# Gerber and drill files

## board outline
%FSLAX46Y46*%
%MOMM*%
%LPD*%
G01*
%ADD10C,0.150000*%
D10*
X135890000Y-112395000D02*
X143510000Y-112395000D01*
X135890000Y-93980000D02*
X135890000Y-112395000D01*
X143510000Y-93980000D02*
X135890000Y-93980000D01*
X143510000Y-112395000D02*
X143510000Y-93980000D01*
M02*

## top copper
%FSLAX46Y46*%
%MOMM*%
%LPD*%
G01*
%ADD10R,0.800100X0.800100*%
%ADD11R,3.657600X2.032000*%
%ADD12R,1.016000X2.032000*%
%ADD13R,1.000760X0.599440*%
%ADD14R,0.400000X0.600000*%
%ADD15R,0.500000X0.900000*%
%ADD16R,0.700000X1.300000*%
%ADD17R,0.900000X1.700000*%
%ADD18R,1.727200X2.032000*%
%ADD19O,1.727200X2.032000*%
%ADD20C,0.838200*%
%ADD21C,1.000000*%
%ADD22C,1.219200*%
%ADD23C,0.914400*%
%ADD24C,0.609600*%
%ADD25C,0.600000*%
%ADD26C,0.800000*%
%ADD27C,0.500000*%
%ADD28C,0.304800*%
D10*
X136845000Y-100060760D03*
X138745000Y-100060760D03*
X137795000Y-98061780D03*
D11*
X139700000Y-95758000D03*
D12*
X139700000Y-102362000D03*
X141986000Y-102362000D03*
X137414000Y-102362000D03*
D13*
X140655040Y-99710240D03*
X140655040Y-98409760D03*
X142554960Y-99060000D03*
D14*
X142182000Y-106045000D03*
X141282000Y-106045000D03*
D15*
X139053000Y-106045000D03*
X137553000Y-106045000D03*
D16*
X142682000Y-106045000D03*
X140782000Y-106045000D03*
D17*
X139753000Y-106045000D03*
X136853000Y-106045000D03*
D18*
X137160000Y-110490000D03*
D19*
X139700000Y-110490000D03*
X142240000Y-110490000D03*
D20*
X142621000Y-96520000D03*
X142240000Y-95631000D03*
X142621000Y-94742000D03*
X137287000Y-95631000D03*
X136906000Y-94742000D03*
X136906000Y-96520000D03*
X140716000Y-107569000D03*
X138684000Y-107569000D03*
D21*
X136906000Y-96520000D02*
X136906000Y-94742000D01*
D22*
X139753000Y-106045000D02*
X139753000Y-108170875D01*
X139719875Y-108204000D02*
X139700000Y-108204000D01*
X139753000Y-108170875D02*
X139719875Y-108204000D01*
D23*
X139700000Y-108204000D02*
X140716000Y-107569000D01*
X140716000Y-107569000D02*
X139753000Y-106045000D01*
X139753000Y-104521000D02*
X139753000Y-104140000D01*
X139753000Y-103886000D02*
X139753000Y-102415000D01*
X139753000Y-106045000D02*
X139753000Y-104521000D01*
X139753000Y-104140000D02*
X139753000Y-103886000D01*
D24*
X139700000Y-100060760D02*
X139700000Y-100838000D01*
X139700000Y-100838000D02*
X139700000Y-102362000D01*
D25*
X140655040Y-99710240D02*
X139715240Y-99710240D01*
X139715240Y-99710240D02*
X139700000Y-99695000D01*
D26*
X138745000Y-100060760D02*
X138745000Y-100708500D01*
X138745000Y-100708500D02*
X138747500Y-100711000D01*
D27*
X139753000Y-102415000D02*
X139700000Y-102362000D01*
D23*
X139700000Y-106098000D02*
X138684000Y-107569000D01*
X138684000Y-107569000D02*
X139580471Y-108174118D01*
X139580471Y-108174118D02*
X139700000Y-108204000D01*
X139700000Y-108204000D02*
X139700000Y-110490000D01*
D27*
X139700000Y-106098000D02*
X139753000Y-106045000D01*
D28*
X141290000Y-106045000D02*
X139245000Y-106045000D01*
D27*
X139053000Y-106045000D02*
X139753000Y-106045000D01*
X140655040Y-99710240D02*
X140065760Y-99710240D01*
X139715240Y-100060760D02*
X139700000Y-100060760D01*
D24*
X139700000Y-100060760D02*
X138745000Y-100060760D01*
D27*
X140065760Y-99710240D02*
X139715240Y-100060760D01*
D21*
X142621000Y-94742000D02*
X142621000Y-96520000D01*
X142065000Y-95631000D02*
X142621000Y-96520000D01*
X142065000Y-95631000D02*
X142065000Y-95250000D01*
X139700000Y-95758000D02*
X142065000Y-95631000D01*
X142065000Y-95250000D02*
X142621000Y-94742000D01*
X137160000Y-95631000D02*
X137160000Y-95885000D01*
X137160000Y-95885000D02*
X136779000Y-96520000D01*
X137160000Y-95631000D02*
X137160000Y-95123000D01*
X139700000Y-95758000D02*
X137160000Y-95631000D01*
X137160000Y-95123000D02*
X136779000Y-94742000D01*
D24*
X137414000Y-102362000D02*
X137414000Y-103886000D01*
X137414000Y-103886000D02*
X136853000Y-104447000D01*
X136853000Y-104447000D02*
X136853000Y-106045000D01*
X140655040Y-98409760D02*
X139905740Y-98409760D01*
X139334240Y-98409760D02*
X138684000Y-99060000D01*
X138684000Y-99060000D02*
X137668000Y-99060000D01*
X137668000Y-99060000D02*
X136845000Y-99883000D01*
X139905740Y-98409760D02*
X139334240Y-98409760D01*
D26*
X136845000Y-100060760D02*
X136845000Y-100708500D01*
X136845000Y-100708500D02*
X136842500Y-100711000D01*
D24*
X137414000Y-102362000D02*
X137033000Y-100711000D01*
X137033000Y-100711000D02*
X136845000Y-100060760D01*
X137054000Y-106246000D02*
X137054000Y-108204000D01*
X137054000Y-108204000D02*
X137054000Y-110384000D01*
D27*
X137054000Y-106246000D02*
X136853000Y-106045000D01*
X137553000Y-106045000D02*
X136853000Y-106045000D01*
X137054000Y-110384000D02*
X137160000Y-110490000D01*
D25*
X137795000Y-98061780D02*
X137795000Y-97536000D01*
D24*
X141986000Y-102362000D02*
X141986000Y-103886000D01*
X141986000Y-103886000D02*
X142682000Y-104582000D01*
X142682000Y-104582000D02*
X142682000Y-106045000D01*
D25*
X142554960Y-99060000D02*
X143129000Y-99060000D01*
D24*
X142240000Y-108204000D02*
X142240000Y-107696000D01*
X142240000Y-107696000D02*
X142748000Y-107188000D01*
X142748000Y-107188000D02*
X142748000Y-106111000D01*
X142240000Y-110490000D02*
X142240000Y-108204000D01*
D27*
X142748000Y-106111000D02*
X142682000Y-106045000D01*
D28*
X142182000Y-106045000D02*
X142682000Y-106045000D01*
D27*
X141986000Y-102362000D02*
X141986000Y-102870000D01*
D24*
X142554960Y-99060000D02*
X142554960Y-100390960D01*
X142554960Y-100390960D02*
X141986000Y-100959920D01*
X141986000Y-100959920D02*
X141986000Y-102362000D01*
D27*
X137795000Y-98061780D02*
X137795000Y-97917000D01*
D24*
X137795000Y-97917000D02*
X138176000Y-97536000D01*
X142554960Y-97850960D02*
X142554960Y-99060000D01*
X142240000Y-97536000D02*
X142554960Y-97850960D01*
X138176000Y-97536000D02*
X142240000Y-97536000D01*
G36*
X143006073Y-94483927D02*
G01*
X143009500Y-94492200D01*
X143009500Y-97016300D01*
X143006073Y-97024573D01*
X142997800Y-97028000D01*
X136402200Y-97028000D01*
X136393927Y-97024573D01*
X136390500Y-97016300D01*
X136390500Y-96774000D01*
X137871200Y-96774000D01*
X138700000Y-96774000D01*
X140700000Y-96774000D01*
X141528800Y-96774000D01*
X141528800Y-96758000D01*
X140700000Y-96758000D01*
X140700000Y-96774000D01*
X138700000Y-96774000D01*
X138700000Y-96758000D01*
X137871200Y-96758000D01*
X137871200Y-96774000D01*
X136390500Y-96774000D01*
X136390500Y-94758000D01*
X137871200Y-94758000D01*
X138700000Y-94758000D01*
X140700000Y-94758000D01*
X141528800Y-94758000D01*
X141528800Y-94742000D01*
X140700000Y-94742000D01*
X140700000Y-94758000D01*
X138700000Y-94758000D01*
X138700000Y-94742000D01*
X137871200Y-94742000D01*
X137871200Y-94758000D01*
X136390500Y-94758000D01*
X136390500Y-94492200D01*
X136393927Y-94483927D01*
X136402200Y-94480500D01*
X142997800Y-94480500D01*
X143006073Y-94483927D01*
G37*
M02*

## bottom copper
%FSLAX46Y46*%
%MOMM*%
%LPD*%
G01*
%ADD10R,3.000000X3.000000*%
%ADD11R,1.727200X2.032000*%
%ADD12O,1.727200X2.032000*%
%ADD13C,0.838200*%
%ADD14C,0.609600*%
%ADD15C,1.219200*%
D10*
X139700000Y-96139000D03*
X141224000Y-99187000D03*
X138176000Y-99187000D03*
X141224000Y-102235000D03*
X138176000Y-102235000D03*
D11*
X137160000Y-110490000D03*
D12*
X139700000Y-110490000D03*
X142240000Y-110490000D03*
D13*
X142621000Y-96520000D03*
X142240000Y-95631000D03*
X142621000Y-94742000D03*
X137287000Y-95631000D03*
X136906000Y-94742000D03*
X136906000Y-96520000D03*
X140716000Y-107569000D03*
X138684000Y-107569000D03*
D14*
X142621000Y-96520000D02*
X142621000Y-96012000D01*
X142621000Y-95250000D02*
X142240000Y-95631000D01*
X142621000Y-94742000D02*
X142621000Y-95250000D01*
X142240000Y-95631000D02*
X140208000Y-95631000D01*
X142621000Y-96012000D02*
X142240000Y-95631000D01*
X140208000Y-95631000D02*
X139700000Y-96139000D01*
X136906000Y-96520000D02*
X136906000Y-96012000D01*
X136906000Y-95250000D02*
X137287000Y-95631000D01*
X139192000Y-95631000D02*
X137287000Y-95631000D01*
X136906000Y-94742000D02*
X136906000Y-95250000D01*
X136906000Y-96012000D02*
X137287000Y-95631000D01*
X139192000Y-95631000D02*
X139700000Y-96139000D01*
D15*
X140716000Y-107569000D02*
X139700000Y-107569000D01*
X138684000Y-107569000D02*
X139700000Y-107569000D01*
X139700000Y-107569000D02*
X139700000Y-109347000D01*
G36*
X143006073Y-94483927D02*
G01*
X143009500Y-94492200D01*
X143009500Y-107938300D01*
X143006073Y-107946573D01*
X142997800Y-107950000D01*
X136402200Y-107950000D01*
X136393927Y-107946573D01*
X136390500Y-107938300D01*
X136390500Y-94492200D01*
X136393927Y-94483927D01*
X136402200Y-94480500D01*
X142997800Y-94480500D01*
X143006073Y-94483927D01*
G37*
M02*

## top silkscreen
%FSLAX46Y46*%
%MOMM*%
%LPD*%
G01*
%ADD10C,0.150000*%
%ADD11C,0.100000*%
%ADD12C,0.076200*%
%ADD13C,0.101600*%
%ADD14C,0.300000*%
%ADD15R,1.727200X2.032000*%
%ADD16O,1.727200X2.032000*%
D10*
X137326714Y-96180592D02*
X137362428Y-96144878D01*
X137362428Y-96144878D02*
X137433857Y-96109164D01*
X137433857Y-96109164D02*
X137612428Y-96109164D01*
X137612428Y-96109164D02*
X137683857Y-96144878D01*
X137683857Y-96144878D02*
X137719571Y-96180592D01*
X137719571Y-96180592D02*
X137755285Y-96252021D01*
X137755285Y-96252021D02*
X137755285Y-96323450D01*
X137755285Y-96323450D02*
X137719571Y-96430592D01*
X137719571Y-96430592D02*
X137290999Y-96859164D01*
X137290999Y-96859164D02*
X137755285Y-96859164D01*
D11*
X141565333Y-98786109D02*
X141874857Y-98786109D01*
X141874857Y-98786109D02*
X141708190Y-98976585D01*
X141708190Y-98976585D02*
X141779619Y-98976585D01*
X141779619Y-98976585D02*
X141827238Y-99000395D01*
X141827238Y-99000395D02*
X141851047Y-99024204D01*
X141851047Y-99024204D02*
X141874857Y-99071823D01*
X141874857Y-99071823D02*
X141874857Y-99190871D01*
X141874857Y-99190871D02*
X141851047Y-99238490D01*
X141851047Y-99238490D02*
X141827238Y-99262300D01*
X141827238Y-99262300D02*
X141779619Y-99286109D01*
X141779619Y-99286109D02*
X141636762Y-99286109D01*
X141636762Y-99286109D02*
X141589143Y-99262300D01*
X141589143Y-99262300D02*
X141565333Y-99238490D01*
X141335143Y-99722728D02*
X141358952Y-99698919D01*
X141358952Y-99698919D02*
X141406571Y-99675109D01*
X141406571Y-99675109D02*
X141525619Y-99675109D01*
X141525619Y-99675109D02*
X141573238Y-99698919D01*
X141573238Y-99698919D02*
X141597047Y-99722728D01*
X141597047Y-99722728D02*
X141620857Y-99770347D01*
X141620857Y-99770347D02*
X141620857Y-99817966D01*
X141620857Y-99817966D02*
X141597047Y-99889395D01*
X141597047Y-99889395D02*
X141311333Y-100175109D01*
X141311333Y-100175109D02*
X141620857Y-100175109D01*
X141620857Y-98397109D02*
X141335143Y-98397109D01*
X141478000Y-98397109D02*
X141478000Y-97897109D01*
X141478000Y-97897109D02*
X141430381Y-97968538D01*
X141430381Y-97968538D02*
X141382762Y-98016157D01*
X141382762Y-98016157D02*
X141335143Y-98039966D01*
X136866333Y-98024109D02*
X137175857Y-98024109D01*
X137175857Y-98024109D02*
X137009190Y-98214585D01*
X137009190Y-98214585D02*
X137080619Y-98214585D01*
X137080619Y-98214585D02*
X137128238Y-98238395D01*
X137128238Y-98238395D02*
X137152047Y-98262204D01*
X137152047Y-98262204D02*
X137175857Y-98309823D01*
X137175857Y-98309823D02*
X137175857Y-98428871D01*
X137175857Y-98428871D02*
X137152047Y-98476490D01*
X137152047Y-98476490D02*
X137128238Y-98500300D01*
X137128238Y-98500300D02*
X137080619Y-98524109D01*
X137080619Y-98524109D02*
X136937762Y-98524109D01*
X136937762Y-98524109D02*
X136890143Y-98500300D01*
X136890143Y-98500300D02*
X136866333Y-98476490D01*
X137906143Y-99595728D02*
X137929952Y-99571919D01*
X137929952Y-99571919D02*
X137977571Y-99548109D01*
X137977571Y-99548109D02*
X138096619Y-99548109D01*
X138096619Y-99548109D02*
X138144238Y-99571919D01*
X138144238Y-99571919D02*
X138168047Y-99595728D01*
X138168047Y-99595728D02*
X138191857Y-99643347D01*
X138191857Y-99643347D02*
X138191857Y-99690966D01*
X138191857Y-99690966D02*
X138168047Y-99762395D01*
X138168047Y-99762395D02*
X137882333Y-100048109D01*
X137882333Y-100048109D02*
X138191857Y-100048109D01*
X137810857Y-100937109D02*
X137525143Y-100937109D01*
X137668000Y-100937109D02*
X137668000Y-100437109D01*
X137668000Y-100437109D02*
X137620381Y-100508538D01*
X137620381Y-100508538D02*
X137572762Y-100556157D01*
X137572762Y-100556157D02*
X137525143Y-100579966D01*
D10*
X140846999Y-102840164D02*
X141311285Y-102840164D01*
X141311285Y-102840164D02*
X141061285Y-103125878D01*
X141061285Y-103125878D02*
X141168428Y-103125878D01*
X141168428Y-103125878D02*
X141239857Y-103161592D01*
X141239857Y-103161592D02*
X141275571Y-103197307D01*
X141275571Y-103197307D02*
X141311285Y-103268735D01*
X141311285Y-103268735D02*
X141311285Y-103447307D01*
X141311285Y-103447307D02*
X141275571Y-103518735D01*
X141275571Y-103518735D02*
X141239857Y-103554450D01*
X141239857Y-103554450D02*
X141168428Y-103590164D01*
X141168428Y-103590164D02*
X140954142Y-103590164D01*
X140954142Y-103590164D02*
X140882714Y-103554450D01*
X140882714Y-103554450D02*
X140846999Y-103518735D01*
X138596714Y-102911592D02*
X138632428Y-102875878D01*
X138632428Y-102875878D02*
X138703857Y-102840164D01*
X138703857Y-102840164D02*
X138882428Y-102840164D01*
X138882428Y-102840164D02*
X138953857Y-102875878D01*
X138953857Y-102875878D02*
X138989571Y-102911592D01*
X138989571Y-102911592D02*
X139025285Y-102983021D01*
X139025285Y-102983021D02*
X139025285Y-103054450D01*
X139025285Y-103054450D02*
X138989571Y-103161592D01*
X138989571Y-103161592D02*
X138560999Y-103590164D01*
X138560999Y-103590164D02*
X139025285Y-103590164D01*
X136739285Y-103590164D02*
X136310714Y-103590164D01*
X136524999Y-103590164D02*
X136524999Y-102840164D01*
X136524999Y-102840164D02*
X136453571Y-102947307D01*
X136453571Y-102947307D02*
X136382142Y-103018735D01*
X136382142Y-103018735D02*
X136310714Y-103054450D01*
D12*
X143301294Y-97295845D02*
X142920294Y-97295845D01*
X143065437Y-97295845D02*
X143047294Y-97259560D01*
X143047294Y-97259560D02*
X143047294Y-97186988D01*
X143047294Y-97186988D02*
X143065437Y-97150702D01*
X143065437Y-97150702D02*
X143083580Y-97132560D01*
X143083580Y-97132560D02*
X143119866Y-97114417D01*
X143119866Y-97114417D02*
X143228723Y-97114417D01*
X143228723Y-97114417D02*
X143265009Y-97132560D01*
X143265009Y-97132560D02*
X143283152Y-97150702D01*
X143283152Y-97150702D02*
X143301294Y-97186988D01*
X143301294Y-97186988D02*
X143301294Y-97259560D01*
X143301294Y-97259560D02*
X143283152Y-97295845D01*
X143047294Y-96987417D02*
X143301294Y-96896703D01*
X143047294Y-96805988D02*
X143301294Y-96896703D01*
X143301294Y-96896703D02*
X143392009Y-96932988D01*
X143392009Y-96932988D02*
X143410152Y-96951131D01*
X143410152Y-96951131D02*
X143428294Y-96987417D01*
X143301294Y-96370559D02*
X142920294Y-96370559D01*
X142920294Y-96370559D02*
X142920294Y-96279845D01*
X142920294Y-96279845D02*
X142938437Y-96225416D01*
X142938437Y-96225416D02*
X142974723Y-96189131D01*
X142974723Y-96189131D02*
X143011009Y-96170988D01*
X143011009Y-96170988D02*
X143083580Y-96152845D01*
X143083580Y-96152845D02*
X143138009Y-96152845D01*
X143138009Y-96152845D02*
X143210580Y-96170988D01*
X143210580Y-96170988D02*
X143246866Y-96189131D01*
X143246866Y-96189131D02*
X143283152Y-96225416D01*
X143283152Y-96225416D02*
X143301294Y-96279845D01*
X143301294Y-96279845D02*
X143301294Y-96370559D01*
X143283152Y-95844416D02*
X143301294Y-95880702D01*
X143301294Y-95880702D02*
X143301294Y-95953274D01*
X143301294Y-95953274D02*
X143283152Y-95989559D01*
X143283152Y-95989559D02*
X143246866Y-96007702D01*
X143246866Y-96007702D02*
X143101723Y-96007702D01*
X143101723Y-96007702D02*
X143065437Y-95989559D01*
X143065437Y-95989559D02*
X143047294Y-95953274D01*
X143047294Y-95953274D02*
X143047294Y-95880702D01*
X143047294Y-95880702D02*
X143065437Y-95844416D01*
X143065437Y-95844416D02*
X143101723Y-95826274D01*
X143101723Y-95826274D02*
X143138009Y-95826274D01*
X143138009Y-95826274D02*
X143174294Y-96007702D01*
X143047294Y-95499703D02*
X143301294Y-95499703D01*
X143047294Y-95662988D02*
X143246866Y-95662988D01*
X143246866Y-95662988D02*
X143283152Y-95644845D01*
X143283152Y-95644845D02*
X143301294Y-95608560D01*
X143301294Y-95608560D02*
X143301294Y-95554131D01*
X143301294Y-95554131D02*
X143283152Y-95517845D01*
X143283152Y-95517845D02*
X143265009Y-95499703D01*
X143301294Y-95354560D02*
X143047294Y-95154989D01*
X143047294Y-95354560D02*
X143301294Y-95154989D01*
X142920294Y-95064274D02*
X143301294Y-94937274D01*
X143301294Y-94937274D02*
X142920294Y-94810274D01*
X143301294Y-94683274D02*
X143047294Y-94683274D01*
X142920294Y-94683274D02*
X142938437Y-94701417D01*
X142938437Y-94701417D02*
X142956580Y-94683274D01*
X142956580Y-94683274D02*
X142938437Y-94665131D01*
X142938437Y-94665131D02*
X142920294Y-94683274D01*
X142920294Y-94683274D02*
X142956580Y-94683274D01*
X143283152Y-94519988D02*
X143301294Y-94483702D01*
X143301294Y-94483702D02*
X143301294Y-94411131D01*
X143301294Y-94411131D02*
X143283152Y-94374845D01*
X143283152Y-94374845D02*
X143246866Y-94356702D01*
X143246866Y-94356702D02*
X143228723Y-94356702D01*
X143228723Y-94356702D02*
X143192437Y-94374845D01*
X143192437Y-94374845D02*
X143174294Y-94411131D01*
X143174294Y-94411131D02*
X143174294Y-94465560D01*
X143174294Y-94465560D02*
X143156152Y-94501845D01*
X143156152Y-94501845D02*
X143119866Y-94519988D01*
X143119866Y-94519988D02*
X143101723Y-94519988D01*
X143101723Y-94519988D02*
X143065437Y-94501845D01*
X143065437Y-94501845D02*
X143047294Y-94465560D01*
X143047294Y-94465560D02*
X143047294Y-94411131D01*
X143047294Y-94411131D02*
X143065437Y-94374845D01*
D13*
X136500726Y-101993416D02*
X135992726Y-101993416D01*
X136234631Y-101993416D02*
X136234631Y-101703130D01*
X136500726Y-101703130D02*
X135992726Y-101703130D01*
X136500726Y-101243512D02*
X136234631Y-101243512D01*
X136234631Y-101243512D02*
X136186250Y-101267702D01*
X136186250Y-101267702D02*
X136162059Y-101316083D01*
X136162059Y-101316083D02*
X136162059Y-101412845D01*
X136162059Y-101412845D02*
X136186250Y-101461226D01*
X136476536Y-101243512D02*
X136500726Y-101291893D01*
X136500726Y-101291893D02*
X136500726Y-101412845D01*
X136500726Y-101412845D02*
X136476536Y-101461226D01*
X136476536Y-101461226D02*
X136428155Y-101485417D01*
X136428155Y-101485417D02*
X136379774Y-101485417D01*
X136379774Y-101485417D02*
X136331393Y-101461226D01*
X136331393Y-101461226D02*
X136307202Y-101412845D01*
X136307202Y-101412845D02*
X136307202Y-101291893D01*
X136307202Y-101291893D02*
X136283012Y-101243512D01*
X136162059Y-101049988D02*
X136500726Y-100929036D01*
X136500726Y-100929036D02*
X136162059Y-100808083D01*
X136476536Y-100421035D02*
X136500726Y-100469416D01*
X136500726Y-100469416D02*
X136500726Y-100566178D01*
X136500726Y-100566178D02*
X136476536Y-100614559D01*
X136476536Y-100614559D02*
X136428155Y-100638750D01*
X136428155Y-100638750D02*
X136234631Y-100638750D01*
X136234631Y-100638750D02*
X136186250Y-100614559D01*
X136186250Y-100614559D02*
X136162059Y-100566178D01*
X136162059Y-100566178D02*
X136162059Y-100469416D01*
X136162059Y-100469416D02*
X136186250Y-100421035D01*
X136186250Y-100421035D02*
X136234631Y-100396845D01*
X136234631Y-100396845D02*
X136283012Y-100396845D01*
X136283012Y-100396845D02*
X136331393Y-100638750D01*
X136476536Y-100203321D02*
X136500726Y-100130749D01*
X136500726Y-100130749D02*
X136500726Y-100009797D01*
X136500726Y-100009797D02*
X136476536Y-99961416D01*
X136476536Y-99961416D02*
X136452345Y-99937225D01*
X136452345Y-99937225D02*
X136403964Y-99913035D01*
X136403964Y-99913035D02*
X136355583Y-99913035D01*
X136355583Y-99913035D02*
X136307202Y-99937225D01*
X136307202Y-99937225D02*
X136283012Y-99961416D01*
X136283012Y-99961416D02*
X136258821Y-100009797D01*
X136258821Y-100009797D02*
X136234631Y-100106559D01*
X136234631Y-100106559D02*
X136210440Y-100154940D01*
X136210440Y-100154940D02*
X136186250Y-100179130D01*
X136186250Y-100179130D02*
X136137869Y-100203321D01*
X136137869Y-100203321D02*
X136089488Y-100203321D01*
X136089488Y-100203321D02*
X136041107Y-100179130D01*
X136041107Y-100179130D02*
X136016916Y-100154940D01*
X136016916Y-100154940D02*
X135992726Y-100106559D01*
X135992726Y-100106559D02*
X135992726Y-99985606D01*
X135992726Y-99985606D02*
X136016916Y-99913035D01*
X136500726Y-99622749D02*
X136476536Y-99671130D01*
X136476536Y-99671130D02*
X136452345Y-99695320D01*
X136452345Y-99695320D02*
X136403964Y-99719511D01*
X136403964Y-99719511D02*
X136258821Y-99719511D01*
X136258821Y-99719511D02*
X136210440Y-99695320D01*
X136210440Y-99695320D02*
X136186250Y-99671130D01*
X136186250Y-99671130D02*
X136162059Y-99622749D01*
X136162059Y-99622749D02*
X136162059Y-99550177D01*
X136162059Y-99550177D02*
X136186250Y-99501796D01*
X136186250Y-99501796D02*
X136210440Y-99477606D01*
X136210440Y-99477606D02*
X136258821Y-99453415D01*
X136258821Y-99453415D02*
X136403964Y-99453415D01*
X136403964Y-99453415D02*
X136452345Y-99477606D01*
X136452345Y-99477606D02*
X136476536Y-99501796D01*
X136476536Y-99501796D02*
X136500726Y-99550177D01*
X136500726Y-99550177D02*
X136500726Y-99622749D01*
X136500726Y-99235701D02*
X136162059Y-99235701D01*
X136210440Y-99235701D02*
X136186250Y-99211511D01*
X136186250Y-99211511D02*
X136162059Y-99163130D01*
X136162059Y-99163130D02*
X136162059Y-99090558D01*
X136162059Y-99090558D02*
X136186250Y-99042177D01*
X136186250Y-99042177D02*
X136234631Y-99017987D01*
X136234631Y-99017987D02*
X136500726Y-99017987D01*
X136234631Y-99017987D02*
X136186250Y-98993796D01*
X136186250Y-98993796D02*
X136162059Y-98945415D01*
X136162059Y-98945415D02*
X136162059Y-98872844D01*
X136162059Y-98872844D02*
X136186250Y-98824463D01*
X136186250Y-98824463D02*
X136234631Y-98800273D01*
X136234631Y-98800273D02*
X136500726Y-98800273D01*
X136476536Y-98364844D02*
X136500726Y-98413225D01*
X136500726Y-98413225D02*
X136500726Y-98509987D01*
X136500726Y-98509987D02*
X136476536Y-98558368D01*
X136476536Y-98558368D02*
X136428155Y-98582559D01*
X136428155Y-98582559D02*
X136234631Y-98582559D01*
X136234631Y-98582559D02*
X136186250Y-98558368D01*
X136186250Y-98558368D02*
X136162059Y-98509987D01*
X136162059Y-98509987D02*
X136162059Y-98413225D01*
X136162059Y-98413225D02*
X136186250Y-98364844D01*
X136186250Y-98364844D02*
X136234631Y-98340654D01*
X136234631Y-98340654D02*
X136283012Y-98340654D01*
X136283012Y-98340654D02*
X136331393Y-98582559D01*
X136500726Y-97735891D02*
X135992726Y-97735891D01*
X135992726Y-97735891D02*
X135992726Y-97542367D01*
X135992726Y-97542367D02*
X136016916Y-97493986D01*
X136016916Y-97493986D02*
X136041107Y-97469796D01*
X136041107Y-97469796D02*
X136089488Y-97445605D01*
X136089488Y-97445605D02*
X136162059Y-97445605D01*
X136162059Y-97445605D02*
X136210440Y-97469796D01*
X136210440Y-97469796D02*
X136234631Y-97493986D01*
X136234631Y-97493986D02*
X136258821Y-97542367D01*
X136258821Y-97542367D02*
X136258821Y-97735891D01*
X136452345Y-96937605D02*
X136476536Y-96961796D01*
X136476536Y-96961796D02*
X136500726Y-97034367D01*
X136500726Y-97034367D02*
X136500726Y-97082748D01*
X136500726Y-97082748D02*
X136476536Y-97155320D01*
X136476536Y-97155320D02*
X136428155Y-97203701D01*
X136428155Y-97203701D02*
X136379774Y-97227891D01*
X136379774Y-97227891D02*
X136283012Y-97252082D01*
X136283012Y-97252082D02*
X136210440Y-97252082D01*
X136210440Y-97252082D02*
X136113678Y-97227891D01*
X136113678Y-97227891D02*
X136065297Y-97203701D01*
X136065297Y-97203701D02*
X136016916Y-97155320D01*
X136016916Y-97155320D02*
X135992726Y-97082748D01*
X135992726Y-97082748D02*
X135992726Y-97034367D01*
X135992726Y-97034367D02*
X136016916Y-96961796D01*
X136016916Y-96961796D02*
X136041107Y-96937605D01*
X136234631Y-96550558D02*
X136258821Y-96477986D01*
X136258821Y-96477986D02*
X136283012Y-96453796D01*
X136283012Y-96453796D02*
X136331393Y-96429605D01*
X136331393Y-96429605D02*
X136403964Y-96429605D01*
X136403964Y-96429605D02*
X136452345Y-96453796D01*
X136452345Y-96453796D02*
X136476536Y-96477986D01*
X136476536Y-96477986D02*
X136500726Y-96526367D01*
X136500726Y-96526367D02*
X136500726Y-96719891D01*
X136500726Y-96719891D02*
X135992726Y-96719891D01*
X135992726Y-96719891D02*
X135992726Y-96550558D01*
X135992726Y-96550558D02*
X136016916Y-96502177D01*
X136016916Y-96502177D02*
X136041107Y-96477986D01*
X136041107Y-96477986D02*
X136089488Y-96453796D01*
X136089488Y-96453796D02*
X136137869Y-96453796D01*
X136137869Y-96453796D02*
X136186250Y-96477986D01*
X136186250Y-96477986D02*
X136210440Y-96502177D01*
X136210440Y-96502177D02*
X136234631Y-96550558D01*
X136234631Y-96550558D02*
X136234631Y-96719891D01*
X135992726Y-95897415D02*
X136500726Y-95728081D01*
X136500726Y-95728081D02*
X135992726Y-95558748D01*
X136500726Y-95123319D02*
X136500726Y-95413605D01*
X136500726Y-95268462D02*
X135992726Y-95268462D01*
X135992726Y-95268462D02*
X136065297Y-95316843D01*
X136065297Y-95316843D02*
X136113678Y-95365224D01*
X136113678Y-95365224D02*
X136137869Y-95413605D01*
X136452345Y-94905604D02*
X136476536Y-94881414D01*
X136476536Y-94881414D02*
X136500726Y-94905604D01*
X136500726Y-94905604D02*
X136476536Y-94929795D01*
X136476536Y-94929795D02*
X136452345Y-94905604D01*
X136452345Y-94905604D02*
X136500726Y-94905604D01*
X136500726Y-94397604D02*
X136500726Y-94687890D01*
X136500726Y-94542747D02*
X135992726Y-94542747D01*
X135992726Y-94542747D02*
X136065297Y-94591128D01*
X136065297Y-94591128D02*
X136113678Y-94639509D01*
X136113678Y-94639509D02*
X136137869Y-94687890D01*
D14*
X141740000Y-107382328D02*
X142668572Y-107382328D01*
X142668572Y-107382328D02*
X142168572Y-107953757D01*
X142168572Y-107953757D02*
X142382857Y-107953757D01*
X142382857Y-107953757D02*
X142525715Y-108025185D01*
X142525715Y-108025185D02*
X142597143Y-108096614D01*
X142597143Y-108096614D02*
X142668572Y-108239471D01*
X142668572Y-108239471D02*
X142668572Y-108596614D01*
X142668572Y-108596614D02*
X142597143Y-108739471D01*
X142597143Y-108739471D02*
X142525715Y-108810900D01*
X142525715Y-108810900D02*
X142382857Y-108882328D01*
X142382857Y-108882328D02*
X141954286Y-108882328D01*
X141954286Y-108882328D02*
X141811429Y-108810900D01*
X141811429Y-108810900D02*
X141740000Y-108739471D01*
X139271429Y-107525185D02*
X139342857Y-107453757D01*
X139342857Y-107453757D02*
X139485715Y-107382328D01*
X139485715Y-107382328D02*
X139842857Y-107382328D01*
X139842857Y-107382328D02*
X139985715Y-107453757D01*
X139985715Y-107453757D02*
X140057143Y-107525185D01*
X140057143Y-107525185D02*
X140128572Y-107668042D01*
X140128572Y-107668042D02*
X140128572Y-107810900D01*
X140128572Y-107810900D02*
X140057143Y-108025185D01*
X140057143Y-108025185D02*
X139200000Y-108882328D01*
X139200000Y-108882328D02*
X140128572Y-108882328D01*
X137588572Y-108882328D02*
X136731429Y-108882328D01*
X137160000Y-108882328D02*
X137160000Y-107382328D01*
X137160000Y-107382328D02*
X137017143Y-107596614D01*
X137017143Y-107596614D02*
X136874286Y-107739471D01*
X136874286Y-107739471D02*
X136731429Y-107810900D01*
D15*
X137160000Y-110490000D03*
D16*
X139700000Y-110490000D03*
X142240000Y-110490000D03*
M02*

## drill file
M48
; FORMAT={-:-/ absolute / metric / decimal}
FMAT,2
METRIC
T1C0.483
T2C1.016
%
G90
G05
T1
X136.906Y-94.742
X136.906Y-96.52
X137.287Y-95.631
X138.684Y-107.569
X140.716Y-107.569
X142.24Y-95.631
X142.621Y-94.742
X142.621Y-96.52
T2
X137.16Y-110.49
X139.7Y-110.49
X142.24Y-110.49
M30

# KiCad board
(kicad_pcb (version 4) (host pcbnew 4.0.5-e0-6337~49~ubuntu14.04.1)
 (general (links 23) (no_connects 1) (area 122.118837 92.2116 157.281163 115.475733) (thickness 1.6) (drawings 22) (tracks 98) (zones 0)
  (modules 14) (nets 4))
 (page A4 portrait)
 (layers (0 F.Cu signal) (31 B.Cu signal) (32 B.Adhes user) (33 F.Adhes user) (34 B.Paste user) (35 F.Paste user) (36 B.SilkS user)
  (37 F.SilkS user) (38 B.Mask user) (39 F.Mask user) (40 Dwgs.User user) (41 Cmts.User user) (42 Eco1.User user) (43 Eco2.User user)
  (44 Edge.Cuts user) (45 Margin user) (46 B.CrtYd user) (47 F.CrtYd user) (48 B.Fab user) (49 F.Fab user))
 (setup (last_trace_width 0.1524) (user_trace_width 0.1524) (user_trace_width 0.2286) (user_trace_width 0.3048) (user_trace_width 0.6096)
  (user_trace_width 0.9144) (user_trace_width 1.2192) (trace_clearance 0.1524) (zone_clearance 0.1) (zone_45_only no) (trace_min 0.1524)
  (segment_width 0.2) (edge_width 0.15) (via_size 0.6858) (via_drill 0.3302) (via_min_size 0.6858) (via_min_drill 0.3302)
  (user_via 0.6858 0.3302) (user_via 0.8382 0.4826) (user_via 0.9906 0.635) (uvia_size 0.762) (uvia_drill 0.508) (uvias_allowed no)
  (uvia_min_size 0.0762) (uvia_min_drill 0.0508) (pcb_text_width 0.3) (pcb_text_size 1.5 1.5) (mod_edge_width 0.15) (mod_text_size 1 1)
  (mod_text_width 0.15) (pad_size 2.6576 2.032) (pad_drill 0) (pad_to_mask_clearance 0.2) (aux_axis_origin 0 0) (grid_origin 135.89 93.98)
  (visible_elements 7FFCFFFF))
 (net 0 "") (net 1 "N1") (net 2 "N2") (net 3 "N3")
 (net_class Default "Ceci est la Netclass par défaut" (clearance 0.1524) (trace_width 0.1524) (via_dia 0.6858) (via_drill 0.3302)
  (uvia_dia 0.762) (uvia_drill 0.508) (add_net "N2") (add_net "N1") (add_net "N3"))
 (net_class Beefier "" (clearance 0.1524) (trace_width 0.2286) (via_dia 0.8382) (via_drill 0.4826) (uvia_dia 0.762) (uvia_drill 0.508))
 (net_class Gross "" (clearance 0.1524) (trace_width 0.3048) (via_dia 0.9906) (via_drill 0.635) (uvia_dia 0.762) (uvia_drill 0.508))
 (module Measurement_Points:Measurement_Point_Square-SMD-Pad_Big (layer B.Cu) (at 139.7 96.139)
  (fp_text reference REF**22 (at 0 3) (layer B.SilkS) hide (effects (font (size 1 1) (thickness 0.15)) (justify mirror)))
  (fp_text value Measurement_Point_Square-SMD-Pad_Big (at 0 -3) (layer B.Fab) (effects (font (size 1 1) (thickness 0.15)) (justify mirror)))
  (pad 1 smd rect (at 0 0) (size 3 3) (layers B.Cu B.Mask) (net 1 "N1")))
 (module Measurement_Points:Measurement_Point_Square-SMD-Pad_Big (layer B.Cu) (at 141.224 99.187)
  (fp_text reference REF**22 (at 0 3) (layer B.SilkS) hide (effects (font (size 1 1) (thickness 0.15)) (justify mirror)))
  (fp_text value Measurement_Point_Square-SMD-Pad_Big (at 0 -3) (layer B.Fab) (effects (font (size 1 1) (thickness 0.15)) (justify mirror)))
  (pad 1 smd rect (at 0 0) (size 3 3) (layers B.Cu B.Mask) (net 1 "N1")))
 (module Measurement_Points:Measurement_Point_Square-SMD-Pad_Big (layer B.Cu) (at 138.176 99.187) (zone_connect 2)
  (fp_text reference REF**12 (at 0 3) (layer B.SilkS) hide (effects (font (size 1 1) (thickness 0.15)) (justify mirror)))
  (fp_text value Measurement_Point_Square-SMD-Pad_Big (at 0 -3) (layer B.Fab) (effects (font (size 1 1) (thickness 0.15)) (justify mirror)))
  (pad 1 smd rect (at 0 0) (size 3 3) (layers B.Cu B.Mask) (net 1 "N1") (zone_connect 2)))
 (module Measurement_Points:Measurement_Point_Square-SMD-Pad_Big (layer B.Cu) (at 141.224 102.235)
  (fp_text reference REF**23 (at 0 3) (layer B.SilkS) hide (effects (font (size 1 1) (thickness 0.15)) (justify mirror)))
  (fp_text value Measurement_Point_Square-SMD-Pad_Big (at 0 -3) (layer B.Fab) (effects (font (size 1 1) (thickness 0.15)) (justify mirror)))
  (pad 1 smd rect (at 0 0) (size 3 3) (layers B.Cu B.Mask) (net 1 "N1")))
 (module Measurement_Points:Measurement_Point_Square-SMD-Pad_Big (layer B.Cu) (at 138.176 102.235) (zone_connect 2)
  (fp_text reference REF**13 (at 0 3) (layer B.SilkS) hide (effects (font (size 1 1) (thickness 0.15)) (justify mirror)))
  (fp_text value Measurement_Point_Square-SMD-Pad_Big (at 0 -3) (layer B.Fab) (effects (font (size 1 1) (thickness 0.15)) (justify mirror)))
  (pad 1 smd rect (at 0 0) (size 3 3) (layers B.Cu B.Mask) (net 1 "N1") (zone_connect 2)))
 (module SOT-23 (layer F.Cu) (at 137.795 99.06)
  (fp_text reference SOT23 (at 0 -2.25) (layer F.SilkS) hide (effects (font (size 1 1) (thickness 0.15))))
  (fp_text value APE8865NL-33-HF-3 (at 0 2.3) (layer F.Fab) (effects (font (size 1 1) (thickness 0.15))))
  (pad 1 smd rect (at -0.95 1.00076) (size 0.8001 0.8001) (layers F.Cu F.Paste F.Mask) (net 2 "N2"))
  (pad 2 smd rect (at 0.95 1.00076) (size 0.8001 0.8001) (layers F.Cu F.Paste F.Mask) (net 1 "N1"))
  (pad 3 smd rect (at 0 -0.99822) (size 0.8001 0.8001) (layers F.Cu F.Paste F.Mask) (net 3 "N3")))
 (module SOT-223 (layer F.Cu) (at 139.7 99.06)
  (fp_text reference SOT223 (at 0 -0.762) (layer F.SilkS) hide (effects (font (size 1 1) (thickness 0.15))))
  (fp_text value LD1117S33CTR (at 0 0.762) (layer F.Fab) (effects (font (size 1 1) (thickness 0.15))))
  (pad 4 smd rect (at 0 -3.302) (size 3.6576 2.032) (layers F.Cu F.Paste F.Mask) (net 1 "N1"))
  (pad 2 smd rect (at 0 3.302) (size 1.016 2.032) (layers F.Cu F.Paste F.Mask) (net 1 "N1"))
  (pad 3 smd rect (at 2.286 3.302) (size 1.016 2.032) (layers F.Cu F.Paste F.Mask) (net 3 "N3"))
  (pad 1 smd rect (at -2.286 3.302) (size 1.016 2.032) (layers F.Cu F.Paste F.Mask) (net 2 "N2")))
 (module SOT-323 (layer F.Cu) (at 141.605 99.06 90)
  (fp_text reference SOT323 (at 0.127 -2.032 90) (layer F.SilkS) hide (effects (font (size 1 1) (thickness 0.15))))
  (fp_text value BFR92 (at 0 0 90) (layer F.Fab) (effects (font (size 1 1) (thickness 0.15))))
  (pad 2 smd rect (at -0.65024 -0.94996 90) (size 0.59944 1.00076) (layers F.Cu F.Paste F.Mask) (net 1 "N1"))
  (pad 1 smd rect (at 0.65024 -0.94996 90) (size 0.59944 1.00076) (layers F.Cu F.Paste F.Mask) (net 2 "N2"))
  (pad 3 smd rect (at 0 0.94996 90) (size 0.59944 1.00076) (layers F.Cu F.Paste F.Mask) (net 3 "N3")))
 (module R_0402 (layer F.Cu) (at 141.732 106.045 180)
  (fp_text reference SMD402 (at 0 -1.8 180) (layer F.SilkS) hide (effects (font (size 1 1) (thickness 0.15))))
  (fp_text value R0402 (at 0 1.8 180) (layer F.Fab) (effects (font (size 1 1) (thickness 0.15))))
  (pad 1 smd rect (at -0.45 0 180) (size 0.4 0.6) (layers F.Cu F.Paste F.Mask) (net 3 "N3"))
  (pad 2 smd rect (at 0.45 0 180) (size 0.4 0.6) (layers F.Cu F.Paste F.Mask) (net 1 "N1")))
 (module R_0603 (layer F.Cu) (at 138.303 106.045 180)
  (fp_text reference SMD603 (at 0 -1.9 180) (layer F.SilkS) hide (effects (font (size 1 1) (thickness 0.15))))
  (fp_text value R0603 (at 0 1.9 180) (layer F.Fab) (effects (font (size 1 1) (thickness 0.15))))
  (pad 1 smd rect (at -0.75 0 180) (size 0.5 0.9) (layers F.Cu F.Paste F.Mask) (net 1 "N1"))
  (pad 2 smd rect (at 0.75 0 180) (size 0.5 0.9) (layers F.Cu F.Paste F.Mask) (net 2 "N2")))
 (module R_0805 (layer F.Cu) (at 141.732 106.045 180)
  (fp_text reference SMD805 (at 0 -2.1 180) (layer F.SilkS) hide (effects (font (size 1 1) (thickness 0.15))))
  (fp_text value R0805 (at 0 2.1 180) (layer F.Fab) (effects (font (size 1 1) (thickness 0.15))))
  (pad 1 smd rect (at -0.95 0 180) (size 0.7 1.3) (layers F.Cu F.Paste F.Mask) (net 3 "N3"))
  (pad 2 smd rect (at 0.95 0 180) (size 0.7 1.3) (layers F.Cu F.Paste F.Mask) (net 1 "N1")))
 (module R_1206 (layer F.Cu) (at 138.303 106.045 180)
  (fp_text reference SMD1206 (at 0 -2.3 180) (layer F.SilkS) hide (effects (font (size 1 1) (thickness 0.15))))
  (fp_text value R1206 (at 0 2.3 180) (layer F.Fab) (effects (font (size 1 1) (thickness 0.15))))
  (pad 1 smd rect (at -1.45 0 180) (size 0.9 1.7) (layers F.Cu F.Paste F.Mask) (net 1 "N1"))
  (pad 2 smd rect (at 1.45 0 180) (size 0.9 1.7) (layers F.Cu F.Paste F.Mask) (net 2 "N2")))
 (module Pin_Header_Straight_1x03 (layer F.Cu) (at 137.16 110.49 90)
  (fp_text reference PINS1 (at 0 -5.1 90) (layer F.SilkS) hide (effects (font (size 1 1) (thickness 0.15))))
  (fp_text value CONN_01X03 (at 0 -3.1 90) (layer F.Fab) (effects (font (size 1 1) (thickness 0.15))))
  (pad 1 thru_hole rect (at 0 0 90) (size 2.032 1.7272) (drill 1.016) (layers *.Cu *.Mask F.SilkS) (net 2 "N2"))
  (pad 2 thru_hole oval (at 0 2.54 90) (size 2.032 1.7272) (drill 1.016) (layers *.Cu *.Mask F.SilkS) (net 1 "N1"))
  (pad 3 thru_hole oval (at 0 5.08 90) (size 2.032 1.7272) (drill 1.016) (layers *.Cu *.Mask F.SilkS) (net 3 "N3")))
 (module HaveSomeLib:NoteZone (layer B.Cu) (at 139.7 108.204)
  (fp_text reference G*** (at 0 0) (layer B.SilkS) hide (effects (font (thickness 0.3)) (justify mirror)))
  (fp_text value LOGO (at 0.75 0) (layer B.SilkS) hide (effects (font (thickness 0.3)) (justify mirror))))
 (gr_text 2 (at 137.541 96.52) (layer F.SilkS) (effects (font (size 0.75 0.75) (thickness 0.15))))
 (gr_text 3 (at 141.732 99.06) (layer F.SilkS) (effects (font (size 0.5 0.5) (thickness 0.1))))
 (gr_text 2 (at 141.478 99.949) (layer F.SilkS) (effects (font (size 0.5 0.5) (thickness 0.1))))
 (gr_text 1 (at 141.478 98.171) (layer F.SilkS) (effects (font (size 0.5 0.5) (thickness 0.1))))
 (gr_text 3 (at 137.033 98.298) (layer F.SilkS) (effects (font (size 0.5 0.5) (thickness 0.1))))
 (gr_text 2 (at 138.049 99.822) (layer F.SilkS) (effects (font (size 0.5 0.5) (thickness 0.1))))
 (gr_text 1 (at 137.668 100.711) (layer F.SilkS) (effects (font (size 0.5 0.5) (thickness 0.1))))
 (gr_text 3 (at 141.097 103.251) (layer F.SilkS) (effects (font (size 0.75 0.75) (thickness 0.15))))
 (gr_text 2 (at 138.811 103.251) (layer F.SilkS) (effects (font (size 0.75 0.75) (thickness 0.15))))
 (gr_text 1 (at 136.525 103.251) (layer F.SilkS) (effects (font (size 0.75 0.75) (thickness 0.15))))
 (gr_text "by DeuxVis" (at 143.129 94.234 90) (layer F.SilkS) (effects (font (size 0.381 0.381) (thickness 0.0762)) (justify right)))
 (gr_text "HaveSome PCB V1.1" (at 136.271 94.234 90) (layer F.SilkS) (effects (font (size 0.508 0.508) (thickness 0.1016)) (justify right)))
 (gr_line (start 135.89 112.395) (end 143.51 112.395) (angle 90) (layer Edge.Cuts) (width 0.15))
 (gr_line (start 135.89 93.98) (end 135.89 112.395) (angle 90) (layer Edge.Cuts) (width 0.15))
 (gr_line (start 143.51 93.98) (end 135.89 93.98) (angle 90) (layer Edge.Cuts) (width 0.15))
 (gr_line (start 143.51 112.395) (end 143.51 93.98) (angle 90) (layer Edge.Cuts) (width 0.15))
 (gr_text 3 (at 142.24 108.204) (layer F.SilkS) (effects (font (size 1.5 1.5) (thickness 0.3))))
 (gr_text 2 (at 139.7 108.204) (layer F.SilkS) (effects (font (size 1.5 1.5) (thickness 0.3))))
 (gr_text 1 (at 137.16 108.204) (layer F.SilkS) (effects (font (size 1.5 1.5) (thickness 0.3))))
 (segment (start 142.621 96.52) (end 142.621 96.012) (width 0.6096) (layer B.Cu) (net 1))
 (via (at 142.621 96.52) (size 0.8382) (drill 0.4826) (layers F.Cu B.Cu) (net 1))
 (via (at 142.24 95.631) (size 0.8382) (drill 0.4826) (layers F.Cu B.Cu) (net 1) (status 30))
 (segment (start 142.621 95.25) (end 142.24 95.631) (width 0.6096) (layer B.Cu) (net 1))
 (via (at 142.621 94.742) (size 0.8382) (drill 0.4826) (layers F.Cu B.Cu) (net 1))
 (segment (start 142.621 94.742) (end 142.621 95.25) (width 0.6096) (layer B.Cu) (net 1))
 (segment (start 142.24 95.631) (end 140.208 95.631) (width 0.6096) (layer B.Cu) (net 1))
 (segment (start 142.621 96.012) (end 142.24 95.631) (width 0.6096) (layer B.Cu) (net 1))
 (segment (start 140.208 95.631) (end 139.7 96.139) (width 0.6096) (layer B.Cu) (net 1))
 (segment (start 136.906 96.52) (end 136.906 96.012) (width 0.6096) (layer B.Cu) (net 1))
 (segment (start 136.906 95.25) (end 137.287 95.631) (width 0.6096) (layer B.Cu) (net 1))
 (segment (start 139.192 95.631) (end 137.287 95.631) (width 0.6096) (layer B.Cu) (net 1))
 (via (at 137.287 95.631) (size 0.8382) (drill 0.4826) (layers F.Cu B.Cu) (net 1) (status 30))
 (segment (start 136.906 96.52) (end 136.906 94.742) (width 1) (layer F.Cu) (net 1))
 (via (at 136.906 94.742) (size 0.8382) (drill 0.4826) (layers F.Cu B.Cu) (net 1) (status 30))
 (via (at 136.906 96.52) (size 0.8382) (drill 0.4826) (layers F.Cu B.Cu) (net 1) (status 30))
 (segment (start 136.906 94.742) (end 136.906 95.25) (width 0.6096) (layer B.Cu) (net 1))
 (segment (start 136.906 96.012) (end 137.287 95.631) (width 0.6096) (layer B.Cu) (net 1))
 (segment (start 139.192 95.631) (end 139.7 96.139) (width 0.6096) (layer B.Cu) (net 1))
 (segment (start 139.753 106.045) (end 139.753 108.170875) (width 1.2192) (layer F.Cu) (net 1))
 (segment (start 139.719875 108.204) (end 139.7 108.204) (width 1.2192) (layer F.Cu) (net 1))
 (segment (start 139.753 108.170875) (end 139.719875 108.204) (width 1.2192) (layer F.Cu) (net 1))
 (segment (start 140.716 107.569) (end 139.7 107.569) (width 1.2192) (layer B.Cu) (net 1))
 (via (at 140.716 107.569) (size 0.8382) (drill 0.4826) (layers F.Cu B.Cu) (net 1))
 (segment (start 138.684 107.569) (end 139.7 107.569) (width 1.2192) (layer B.Cu) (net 1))
 (via (at 138.684 107.569) (size 0.8382) (drill 0.4826) (layers F.Cu B.Cu) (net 1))
 (segment (start 139.7 107.569) (end 139.7 109.347) (width 1.2192) (layer B.Cu) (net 1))
 (segment (start 139.7 108.204) (end 140.716 107.569) (width 0.9144) (layer F.Cu) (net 1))
 (segment (start 140.716 107.569) (end 139.753 106.045) (width 0.9144) (layer F.Cu) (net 1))
 (segment (start 139.753 104.521) (end 139.753 104.14) (width 0.9144) (layer F.Cu) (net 1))
 (segment (start 139.753 103.886) (end 139.753 102.415) (width 0.9144) (layer F.Cu) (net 1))
 (segment (start 139.753 106.045) (end 139.753 104.521) (width 0.9144) (layer F.Cu) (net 1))
 (segment (start 139.753 104.14) (end 139.753 103.886) (width 0.9144) (layer F.Cu) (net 1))
 (segment (start 139.7 100.06076) (end 139.7 100.838) (width 0.6096) (layer F.Cu) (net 1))
 (segment (start 139.7 100.838) (end 139.7 102.362) (width 0.6096) (layer F.Cu) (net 1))
 (segment (start 140.65504 99.71024) (end 139.71524 99.71024) (width 0.6) (layer F.Cu) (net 1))
 (segment (start 139.71524 99.71024) (end 139.7 99.695) (width 0.6) (layer F.Cu) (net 1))
 (segment (start 138.745 100.06076) (end 138.745 100.7085) (width 0.8) (layer F.Cu) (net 1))
 (segment (start 138.745 100.7085) (end 138.7475 100.711) (width 0.8) (layer F.Cu) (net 1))
 (segment (start 139.753 102.415) (end 139.7 102.362) (width 0.5) (layer F.Cu) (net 1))
 (segment (start 139.7 106.098) (end 138.684 107.569) (width 0.9144) (layer F.Cu) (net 1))
 (segment (start 138.684 107.569) (end 139.580471 108.174118) (width 0.9144) (layer F.Cu) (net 1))
 (segment (start 139.580471 108.174118) (end 139.7 108.204) (width 0.9144) (layer F.Cu) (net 1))
 (segment (start 139.7 108.204) (end 139.7 110.49) (width 0.9144) (layer F.Cu) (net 1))
 (segment (start 139.7 106.098) (end 139.753 106.045) (width 0.5) (layer F.Cu) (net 1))
 (segment (start 141.29 106.045) (end 139.245 106.045) (width 0.3048) (layer F.Cu) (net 1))
 (segment (start 139.053 106.045) (end 139.753 106.045) (width 0.5) (layer F.Cu) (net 1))
 (segment (start 140.65504 99.71024) (end 140.06576 99.71024) (width 0.5) (layer F.Cu) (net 1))
 (segment (start 139.71524 100.06076) (end 139.7 100.06076) (width 0.5) (layer F.Cu) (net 1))
 (segment (start 139.7 100.06076) (end 138.745 100.06076) (width 0.6096) (layer F.Cu) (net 1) (status 20))
 (segment (start 140.06576 99.71024) (end 139.71524 100.06076) (width 0.5) (layer F.Cu) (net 1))
 (segment (start 142.621 94.742) (end 142.621 96.52) (width 1) (layer F.Cu) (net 1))
 (segment (start 142.065 95.631) (end 142.621 96.52) (width 1) (layer F.Cu) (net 1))
 (segment (start 142.065 95.631) (end 142.065 95.25) (width 1) (layer F.Cu) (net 1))
 (segment (start 139.7 95.758) (end 142.065 95.631) (width 1) (layer F.Cu) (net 1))
 (segment (start 142.065 95.25) (end 142.621 94.742) (width 1) (layer F.Cu) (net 1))
 (segment (start 137.16 95.631) (end 137.16 95.885) (width 1) (layer F.Cu) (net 1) (status 30))
 (segment (start 137.16 95.885) (end 136.779 96.52) (width 1) (layer F.Cu) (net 1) (status 30))
 (segment (start 137.16 95.631) (end 137.16 95.123) (width 1) (layer F.Cu) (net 1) (status 30))
 (segment (start 139.7 95.758) (end 137.16 95.631) (width 1) (layer F.Cu) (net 1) (status 20))
 (segment (start 137.16 95.123) (end 136.779 94.742) (width 1) (layer F.Cu) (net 1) (status 30))
 (segment (start 137.414 102.362) (end 137.414 103.886) (width 0.6096) (layer F.Cu) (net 2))
 (segment (start 137.414 103.886) (end 136.853 104.447) (width 0.6096) (layer F.Cu) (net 2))
 (segment (start 136.853 104.447) (end 136.853 106.045) (width 0.6096) (layer F.Cu) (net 2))
 (segment (start 140.65504 98.40976) (end 139.90574 98.40976) (width 0.6096) (layer F.Cu) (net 2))
 (segment (start 139.33424 98.40976) (end 138.684 99.06) (width 0.6096) (layer F.Cu) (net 2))
 (segment (start 138.684 99.06) (end 137.668 99.06) (width 0.6096) (layer F.Cu) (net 2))
 (segment (start 137.668 99.06) (end 136.845 99.883) (width 0.6096) (layer F.Cu) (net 2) (status 20))
 (segment (start 139.90574 98.40976) (end 139.33424 98.40976) (width 0.6096) (layer F.Cu) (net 2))
 (segment (start 136.845 100.06076) (end 136.845 100.7085) (width 0.8) (layer F.Cu) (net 2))
 (segment (start 136.845 100.7085) (end 136.8425 100.711) (width 0.8) (layer F.Cu) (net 2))
 (segment (start 137.414 102.362) (end 137.033 100.711) (width 0.6096) (layer F.Cu) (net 2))
 (segment (start 137.033 100.711) (end 136.845 100.06076) (width 0.6096) (layer F.Cu) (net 2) (status 20))
 (segment (start 137.054 106.246) (end 137.054 108.204) (width 0.6096) (layer F.Cu) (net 2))
 (segment (start 137.054 108.204) (end 137.054 110.384) (width 0.6096) (layer F.Cu) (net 2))
 (segment (start 137.054 106.246) (end 136.853 106.045) (width 0.5) (layer F.Cu) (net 2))
 (segment (start 137.553 106.045) (end 136.853 106.045) (width 0.5) (layer F.Cu) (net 2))
 (segment (start 137.054 110.384) (end 137.16 110.49) (width 0.5) (layer F.Cu) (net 2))
 (segment (start 137.795 98.06178) (end 137.795 97.536) (width 0.6) (layer F.Cu) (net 3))
 (segment (start 141.986 102.362) (end 141.986 103.886) (width 0.6096) (layer F.Cu) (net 3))
 (segment (start 141.986 103.886) (end 142.682 104.582) (width 0.6096) (layer F.Cu) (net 3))
 (segment (start 142.682 104.582) (end 142.682 106.045) (width 0.6096) (layer F.Cu) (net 3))
 (segment (start 142.55496 99.06) (end 143.129 99.06) (width 0.6) (layer F.Cu) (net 3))
 (segment (start 142.24 108.204) (end 142.24 107.696) (width 0.6096) (layer F.Cu) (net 3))
 (segment (start 142.24 107.696) (end 142.748 107.188) (width 0.6096) (layer F.Cu) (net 3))
 (segment (start 142.748 107.188) (end 142.748 106.111) (width 0.6096) (layer F.Cu) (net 3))
 (segment (start 142.24 110.49) (end 142.24 108.204) (width 0.6096) (layer F.Cu) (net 3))
 (segment (start 142.748 106.111) (end 142.682 106.045) (width 0.5) (layer F.Cu) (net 3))
 (segment (start 142.182 106.045) (end 142.682 106.045) (width 0.3048) (layer F.Cu) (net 3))
 (segment (start 141.986 102.362) (end 141.986 102.87) (width 0.5) (layer F.Cu) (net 3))
 (segment (start 142.55496 99.06) (end 142.55496 100.39096) (width 0.6096) (layer F.Cu) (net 3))
 (segment (start 142.55496 100.39096) (end 141.986 100.95992) (width 0.6096) (layer F.Cu) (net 3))
 (segment (start 141.986 100.95992) (end 141.986 102.362) (width 0.6096) (layer F.Cu) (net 3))
 (segment (start 137.795 98.06178) (end 137.795 97.917) (width 0.5) (layer F.Cu) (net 3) (status 30))
 (segment (start 137.795 97.917) (end 138.176 97.536) (width 0.6096) (layer F.Cu) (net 3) (status 10))
 (segment (start 142.55496 97.85096) (end 142.55496 99.06) (width 0.6096) (layer F.Cu) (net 3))
 (segment (start 142.24 97.536) (end 142.55496 97.85096) (width 0.6096) (layer F.Cu) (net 3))
 (segment (start 138.176 97.536) (end 142.24 97.536) (width 0.6096) (layer F.Cu) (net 3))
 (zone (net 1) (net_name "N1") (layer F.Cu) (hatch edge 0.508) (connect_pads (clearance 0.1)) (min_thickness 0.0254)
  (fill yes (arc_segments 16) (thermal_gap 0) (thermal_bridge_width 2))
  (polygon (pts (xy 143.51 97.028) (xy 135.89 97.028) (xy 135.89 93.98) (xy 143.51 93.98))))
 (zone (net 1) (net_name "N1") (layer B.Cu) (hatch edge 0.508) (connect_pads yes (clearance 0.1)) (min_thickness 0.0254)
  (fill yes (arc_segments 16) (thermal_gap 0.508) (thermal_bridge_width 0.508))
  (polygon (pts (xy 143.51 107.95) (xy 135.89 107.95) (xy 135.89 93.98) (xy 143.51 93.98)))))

